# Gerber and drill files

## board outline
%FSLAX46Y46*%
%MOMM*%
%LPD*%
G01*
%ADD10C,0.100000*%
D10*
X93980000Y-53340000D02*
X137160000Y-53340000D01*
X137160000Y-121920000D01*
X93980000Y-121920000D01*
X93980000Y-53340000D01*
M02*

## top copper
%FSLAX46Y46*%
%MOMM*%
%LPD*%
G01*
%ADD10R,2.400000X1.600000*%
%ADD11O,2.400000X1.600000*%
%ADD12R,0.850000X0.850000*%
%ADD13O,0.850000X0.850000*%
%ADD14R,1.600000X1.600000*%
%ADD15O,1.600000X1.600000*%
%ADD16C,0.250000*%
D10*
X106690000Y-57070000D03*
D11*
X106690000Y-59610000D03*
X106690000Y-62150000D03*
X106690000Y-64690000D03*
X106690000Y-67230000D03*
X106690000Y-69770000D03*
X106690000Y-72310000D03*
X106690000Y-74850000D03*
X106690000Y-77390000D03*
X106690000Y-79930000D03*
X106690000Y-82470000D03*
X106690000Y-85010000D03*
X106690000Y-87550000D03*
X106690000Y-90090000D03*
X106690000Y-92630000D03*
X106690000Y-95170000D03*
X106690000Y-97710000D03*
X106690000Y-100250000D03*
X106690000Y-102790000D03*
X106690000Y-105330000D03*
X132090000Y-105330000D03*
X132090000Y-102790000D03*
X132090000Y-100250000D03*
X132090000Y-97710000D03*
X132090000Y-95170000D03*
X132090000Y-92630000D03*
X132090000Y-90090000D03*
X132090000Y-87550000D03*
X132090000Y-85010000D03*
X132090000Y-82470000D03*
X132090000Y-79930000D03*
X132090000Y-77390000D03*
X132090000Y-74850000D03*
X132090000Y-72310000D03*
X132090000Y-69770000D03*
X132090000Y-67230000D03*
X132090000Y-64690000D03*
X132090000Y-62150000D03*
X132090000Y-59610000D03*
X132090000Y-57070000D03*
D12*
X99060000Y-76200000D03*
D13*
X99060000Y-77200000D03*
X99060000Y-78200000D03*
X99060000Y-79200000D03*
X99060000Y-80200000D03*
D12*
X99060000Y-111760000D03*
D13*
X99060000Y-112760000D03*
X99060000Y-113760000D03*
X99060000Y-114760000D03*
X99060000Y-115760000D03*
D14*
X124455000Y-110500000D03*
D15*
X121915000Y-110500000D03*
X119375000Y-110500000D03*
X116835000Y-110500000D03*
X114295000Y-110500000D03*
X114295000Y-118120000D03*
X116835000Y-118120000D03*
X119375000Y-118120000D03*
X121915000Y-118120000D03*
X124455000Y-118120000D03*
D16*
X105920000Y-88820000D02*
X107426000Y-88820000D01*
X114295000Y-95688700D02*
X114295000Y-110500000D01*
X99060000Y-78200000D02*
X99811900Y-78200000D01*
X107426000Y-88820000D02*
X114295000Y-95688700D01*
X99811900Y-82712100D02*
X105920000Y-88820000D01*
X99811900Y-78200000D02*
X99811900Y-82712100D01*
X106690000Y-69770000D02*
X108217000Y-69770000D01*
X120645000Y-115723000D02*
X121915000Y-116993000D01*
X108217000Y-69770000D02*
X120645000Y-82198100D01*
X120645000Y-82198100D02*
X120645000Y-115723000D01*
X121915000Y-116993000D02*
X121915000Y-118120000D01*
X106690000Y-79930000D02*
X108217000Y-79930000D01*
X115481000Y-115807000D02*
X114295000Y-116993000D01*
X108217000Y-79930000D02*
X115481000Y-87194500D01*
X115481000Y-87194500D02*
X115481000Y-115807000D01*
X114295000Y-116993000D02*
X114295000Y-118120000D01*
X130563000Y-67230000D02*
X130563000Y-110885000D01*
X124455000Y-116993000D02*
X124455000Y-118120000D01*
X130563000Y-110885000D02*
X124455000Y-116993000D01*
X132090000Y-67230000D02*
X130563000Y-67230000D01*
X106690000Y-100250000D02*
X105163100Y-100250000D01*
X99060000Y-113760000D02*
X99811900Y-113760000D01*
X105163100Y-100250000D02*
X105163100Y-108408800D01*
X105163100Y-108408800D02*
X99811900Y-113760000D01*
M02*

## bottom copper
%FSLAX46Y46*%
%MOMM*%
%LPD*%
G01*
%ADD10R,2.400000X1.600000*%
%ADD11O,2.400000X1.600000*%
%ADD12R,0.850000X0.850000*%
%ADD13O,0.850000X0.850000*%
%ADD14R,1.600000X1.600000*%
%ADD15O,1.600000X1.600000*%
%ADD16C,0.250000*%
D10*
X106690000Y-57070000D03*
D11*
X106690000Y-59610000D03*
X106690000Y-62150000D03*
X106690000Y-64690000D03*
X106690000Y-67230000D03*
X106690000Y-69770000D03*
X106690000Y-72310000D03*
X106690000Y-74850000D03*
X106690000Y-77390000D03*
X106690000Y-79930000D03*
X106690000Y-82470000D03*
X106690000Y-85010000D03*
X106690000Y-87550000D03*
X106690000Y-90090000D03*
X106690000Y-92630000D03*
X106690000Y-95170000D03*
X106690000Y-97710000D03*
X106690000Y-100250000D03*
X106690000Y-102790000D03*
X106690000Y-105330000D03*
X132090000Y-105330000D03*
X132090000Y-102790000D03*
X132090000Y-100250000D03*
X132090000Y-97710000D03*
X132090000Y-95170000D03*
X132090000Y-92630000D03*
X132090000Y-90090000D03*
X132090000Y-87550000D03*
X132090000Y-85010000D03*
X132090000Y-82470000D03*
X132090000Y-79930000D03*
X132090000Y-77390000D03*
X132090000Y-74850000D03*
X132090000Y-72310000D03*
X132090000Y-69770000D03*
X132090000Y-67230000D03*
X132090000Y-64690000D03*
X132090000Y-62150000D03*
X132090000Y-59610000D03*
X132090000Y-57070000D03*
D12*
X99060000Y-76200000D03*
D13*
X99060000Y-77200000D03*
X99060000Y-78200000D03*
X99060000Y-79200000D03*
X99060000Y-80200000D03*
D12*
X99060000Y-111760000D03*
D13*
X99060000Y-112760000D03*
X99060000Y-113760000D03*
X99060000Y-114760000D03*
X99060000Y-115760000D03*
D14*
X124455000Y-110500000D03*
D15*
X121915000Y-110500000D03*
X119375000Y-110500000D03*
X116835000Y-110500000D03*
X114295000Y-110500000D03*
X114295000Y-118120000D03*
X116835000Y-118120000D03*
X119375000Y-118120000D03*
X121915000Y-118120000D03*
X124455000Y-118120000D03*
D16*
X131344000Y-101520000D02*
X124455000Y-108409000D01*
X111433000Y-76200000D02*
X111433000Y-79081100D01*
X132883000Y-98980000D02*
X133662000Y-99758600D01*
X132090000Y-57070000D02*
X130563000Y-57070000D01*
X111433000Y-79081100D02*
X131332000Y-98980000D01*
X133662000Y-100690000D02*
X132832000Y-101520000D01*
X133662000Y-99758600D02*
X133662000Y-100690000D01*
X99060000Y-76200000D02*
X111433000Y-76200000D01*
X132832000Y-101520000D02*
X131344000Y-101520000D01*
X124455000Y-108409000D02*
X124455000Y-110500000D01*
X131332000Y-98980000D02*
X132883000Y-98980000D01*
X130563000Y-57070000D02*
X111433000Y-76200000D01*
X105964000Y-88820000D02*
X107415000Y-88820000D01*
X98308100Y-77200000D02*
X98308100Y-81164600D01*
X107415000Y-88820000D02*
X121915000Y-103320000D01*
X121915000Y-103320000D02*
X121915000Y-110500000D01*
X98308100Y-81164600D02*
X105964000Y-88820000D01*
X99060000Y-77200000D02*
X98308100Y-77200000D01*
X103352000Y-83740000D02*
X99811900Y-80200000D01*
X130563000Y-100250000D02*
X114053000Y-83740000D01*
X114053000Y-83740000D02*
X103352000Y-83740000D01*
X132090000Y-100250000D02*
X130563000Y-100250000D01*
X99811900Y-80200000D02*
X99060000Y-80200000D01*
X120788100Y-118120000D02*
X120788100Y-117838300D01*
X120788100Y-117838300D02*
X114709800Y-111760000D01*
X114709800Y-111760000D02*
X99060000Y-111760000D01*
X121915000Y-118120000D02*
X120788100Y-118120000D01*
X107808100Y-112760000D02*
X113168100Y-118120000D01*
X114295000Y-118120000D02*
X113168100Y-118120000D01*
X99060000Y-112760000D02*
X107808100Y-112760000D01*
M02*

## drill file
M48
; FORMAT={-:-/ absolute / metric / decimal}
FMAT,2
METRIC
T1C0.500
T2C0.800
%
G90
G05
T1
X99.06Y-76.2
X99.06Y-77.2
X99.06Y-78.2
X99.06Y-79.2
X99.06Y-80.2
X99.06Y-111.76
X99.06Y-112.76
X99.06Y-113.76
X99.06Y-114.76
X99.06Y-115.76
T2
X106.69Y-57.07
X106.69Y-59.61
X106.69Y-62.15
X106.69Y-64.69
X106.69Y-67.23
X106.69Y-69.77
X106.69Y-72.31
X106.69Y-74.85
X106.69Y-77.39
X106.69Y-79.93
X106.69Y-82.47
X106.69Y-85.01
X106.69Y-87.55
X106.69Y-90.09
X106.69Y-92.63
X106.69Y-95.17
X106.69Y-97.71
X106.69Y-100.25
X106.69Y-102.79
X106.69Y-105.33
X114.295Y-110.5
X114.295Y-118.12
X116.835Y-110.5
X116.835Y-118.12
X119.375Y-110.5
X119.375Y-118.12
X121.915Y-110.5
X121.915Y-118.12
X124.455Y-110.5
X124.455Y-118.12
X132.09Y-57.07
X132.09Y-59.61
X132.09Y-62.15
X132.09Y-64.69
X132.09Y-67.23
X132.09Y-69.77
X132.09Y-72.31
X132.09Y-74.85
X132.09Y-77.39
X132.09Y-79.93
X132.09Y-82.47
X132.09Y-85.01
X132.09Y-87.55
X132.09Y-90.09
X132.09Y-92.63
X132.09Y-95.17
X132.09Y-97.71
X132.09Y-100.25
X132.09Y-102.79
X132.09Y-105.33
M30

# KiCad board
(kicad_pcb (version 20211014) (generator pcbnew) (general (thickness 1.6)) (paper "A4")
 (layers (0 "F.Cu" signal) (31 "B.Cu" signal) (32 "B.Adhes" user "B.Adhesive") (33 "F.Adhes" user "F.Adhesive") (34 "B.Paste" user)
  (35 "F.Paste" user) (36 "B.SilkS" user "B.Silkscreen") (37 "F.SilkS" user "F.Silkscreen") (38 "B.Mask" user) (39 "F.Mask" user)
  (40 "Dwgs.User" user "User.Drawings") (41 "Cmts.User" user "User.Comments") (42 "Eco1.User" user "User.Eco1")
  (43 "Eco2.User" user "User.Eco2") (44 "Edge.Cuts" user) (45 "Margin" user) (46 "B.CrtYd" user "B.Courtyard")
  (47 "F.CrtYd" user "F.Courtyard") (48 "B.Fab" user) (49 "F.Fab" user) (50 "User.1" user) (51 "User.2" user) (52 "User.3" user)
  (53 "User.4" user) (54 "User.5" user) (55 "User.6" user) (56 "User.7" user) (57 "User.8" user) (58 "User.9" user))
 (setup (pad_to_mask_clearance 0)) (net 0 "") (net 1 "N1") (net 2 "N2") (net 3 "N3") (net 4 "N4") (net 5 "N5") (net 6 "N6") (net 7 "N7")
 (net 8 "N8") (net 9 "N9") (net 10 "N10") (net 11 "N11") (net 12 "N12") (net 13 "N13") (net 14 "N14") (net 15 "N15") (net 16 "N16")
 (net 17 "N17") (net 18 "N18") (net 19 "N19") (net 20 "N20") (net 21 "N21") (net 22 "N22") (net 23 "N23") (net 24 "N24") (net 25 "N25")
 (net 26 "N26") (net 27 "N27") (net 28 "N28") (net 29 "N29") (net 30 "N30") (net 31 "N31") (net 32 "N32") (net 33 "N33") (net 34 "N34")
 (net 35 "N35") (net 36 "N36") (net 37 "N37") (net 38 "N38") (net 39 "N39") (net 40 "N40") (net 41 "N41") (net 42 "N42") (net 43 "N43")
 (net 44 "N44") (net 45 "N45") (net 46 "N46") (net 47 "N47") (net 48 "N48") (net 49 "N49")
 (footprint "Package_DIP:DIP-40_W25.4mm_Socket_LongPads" (layer "F.Cu") (at 106.69 57.07)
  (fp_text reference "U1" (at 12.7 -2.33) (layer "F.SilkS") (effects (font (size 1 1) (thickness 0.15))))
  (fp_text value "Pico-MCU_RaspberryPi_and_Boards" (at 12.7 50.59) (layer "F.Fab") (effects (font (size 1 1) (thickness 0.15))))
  (pad "1" thru_hole rect (at 0 0) (size 2.4 1.6) (drill 0.8) (layers *.Cu *.Mask) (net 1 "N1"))
  (pad "2" thru_hole oval (at 0 2.54) (size 2.4 1.6) (drill 0.8) (layers *.Cu *.Mask) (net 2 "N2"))
  (pad "3" thru_hole oval (at 0 5.08) (size 2.4 1.6) (drill 0.8) (layers *.Cu *.Mask) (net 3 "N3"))
  (pad "4" thru_hole oval (at 0 7.62) (size 2.4 1.6) (drill 0.8) (layers *.Cu *.Mask) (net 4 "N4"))
  (pad "5" thru_hole oval (at 0 10.16) (size 2.4 1.6) (drill 0.8) (layers *.Cu *.Mask) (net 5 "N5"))
  (pad "6" thru_hole oval (at 0 12.7) (size 2.4 1.6) (drill 0.8) (layers *.Cu *.Mask) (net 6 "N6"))
  (pad "7" thru_hole oval (at 0 15.24) (size 2.4 1.6) (drill 0.8) (layers *.Cu *.Mask) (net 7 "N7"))
  (pad "8" thru_hole oval (at 0 17.78) (size 2.4 1.6) (drill 0.8) (layers *.Cu *.Mask) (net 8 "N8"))
  (pad "9" thru_hole oval (at 0 20.32) (size 2.4 1.6) (drill 0.8) (layers *.Cu *.Mask) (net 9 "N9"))
  (pad "10" thru_hole oval (at 0 22.86) (size 2.4 1.6) (drill 0.8) (layers *.Cu *.Mask) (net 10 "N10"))
  (pad "11" thru_hole oval (at 0 25.4) (size 2.4 1.6) (drill 0.8) (layers *.Cu *.Mask) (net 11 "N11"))
  (pad "12" thru_hole oval (at 0 27.94) (size 2.4 1.6) (drill 0.8) (layers *.Cu *.Mask) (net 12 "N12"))
  (pad "13" thru_hole oval (at 0 30.48) (size 2.4 1.6) (drill 0.8) (layers *.Cu *.Mask) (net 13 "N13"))
  (pad "14" thru_hole oval (at 0 33.02) (size 2.4 1.6) (drill 0.8) (layers *.Cu *.Mask) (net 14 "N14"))
  (pad "15" thru_hole oval (at 0 35.56) (size 2.4 1.6) (drill 0.8) (layers *.Cu *.Mask) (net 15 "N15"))
  (pad "16" thru_hole oval (at 0 38.1) (size 2.4 1.6) (drill 0.8) (layers *.Cu *.Mask) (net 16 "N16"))
  (pad "17" thru_hole oval (at 0 40.64) (size 2.4 1.6) (drill 0.8) (layers *.Cu *.Mask) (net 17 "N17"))
  (pad "18" thru_hole oval (at 0 43.18) (size 2.4 1.6) (drill 0.8) (layers *.Cu *.Mask) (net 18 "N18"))
  (pad "19" thru_hole oval (at 0 45.72) (size 2.4 1.6) (drill 0.8) (layers *.Cu *.Mask) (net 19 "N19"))
  (pad "20" thru_hole oval (at 0 48.26) (size 2.4 1.6) (drill 0.8) (layers *.Cu *.Mask) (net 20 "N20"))
  (pad "21" thru_hole oval (at 25.4 48.26) (size 2.4 1.6) (drill 0.8) (layers *.Cu *.Mask) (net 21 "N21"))
  (pad "22" thru_hole oval (at 25.4 45.72) (size 2.4 1.6) (drill 0.8) (layers *.Cu *.Mask) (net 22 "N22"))
  (pad "23" thru_hole oval (at 25.4 43.18) (size 2.4 1.6) (drill 0.8) (layers *.Cu *.Mask) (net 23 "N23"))
  (pad "24" thru_hole oval (at 25.4 40.64) (size 2.4 1.6) (drill 0.8) (layers *.Cu *.Mask) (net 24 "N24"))
  (pad "25" thru_hole oval (at 25.4 38.1) (size 2.4 1.6) (drill 0.8) (layers *.Cu *.Mask) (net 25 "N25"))
  (pad "26" thru_hole oval (at 25.4 35.56) (size 2.4 1.6) (drill 0.8) (layers *.Cu *.Mask) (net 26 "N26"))
  (pad "27" thru_hole oval (at 25.4 33.02) (size 2.4 1.6) (drill 0.8) (layers *.Cu *.Mask) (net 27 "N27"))
  (pad "28" thru_hole oval (at 25.4 30.48) (size 2.4 1.6) (drill 0.8) (layers *.Cu *.Mask) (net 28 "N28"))
  (pad "29" thru_hole oval (at 25.4 27.94) (size 2.4 1.6) (drill 0.8) (layers *.Cu *.Mask) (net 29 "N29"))
  (pad "30" thru_hole oval (at 25.4 25.4) (size 2.4 1.6) (drill 0.8) (layers *.Cu *.Mask) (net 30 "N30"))
  (pad "31" thru_hole oval (at 25.4 22.86) (size 2.4 1.6) (drill 0.8) (layers *.Cu *.Mask) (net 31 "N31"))
  (pad "32" thru_hole oval (at 25.4 20.32) (size 2.4 1.6) (drill 0.8) (layers *.Cu *.Mask) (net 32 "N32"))
  (pad "33" thru_hole oval (at 25.4 17.78) (size 2.4 1.6) (drill 0.8) (layers *.Cu *.Mask) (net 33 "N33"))
  (pad "34" thru_hole oval (at 25.4 15.24) (size 2.4 1.6) (drill 0.8) (layers *.Cu *.Mask) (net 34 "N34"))
  (pad "35" thru_hole oval (at 25.4 12.7) (size 2.4 1.6) (drill 0.8) (layers *.Cu *.Mask) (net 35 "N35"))
  (pad "36" thru_hole oval (at 25.4 10.16) (size 2.4 1.6) (drill 0.8) (layers *.Cu *.Mask) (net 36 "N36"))
  (pad "37" thru_hole oval (at 25.4 7.62) (size 2.4 1.6) (drill 0.8) (layers *.Cu *.Mask) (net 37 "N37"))
  (pad "38" thru_hole oval (at 25.4 5.08) (size 2.4 1.6) (drill 0.8) (layers *.Cu *.Mask) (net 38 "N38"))
  (pad "39" thru_hole oval (at 25.4 2.54) (size 2.4 1.6) (drill 0.8) (layers *.Cu *.Mask) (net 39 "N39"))
  (pad "40" thru_hole oval (at 25.4 0) (size 2.4 1.6) (drill 0.8) (layers *.Cu *.Mask) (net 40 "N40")))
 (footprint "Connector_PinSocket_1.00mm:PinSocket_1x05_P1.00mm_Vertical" (layer "F.Cu") (at 99.06 76.2)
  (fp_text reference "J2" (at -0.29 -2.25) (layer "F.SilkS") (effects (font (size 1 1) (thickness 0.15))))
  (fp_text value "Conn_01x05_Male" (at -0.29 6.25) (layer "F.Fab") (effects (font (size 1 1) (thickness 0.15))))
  (pad "1" thru_hole rect (at 0 0) (size 0.85 0.85) (drill 0.5) (layers *.Cu *.Mask) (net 40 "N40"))
  (pad "2" thru_hole oval (at 0 1) (size 0.85 0.85) (drill 0.5) (layers *.Cu *.Mask) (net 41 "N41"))
  (pad "3" thru_hole oval (at 0 2) (size 0.85 0.85) (drill 0.5) (layers *.Cu *.Mask) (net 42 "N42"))
  (pad "4" thru_hole oval (at 0 3) (size 0.85 0.85) (drill 0.5) (layers *.Cu *.Mask) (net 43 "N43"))
  (pad "5" thru_hole oval (at 0 4) (size 0.85 0.85) (drill 0.5) (layers *.Cu *.Mask) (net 23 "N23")))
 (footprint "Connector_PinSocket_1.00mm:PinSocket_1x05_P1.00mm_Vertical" (layer "F.Cu") (at 99.06 111.76)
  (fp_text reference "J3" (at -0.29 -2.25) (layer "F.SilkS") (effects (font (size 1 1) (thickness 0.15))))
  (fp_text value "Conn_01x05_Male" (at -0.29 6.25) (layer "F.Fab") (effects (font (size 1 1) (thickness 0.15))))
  (pad "1" thru_hole rect (at 0 0) (size 0.85 0.85) (drill 0.5) (layers *.Cu *.Mask) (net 6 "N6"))
  (pad "2" thru_hole oval (at 0 1) (size 0.85 0.85) (drill 0.5) (layers *.Cu *.Mask) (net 10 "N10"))
  (pad "3" thru_hole oval (at 0 2) (size 0.85 0.85) (drill 0.5) (layers *.Cu *.Mask) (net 18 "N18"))
  (pad "4" thru_hole oval (at 0 3) (size 0.85 0.85) (drill 0.5) (layers *.Cu *.Mask) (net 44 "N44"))
  (pad "5" thru_hole oval (at 0 4) (size 0.85 0.85) (drill 0.5) (layers *.Cu *.Mask) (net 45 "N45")))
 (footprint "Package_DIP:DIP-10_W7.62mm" (layer "F.Cu") (at 124.455 110.5 -90)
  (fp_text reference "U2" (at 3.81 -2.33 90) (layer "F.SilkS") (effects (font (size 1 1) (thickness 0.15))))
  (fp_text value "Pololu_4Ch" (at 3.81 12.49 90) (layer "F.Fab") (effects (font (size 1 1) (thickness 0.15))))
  (pad "1" thru_hole rect (at 0 0 270) (size 1.6 1.6) (drill 0.8) (layers *.Cu *.Mask) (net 40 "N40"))
  (pad "2" thru_hole oval (at 0 2.54 270) (size 1.6 1.6) (drill 0.8) (layers *.Cu *.Mask) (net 41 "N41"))
  (pad "3" thru_hole oval (at 0 5.08 270) (size 1.6 1.6) (drill 0.8) (layers *.Cu *.Mask) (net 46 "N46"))
  (pad "4" thru_hole oval (at 0 7.62 270) (size 1.6 1.6) (drill 0.8) (layers *.Cu *.Mask) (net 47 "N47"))
  (pad "5" thru_hole oval (at 0 10.16 270) (size 1.6 1.6) (drill 0.8) (layers *.Cu *.Mask) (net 42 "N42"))
  (pad "6" thru_hole oval (at 7.62 10.16 270) (size 1.6 1.6) (drill 0.8) (layers *.Cu *.Mask) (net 10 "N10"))
  (pad "7" thru_hole oval (at 7.62 7.62 270) (size 1.6 1.6) (drill 0.8) (layers *.Cu *.Mask) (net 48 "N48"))
  (pad "8" thru_hole oval (at 7.62 5.08 270) (size 1.6 1.6) (drill 0.8) (layers *.Cu *.Mask) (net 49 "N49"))
  (pad "9" thru_hole oval (at 7.62 2.54 270) (size 1.6 1.6) (drill 0.8) (layers *.Cu *.Mask) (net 6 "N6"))
  (pad "10" thru_hole oval (at 7.62 0 270) (size 1.6 1.6) (drill 0.8) (layers *.Cu *.Mask) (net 36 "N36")))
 (gr_rect (start 93.98 53.34) (end 137.16 121.92) (layer "Edge.Cuts") (width 0.1) (fill none))
 (segment (start 131.344 101.52) (end 124.455 108.409) (width 0.25) (layer "B.Cu") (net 40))
 (segment (start 111.433 76.2) (end 111.433 79.0811) (width 0.25) (layer "B.Cu") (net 40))
 (segment (start 132.883 98.98) (end 133.662 99.7586) (width 0.25) (layer "B.Cu") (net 40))
 (segment (start 132.09 57.07) (end 130.563 57.07) (width 0.25) (layer "B.Cu") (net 40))
 (segment (start 111.433 79.0811) (end 131.332 98.98) (width 0.25) (layer "B.Cu") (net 40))
 (segment (start 133.662 100.69) (end 132.832 101.52) (width 0.25) (layer "B.Cu") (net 40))
 (segment (start 133.662 99.7586) (end 133.662 100.69) (width 0.25) (layer "B.Cu") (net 40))
 (segment (start 99.06 76.2) (end 111.433 76.2) (width 0.25) (layer "B.Cu") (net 40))
 (segment (start 132.832 101.52) (end 131.344 101.52) (width 0.25) (layer "B.Cu") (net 40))
 (segment (start 124.455 108.409) (end 124.455 110.5) (width 0.25) (layer "B.Cu") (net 40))
 (segment (start 131.332 98.98) (end 132.883 98.98) (width 0.25) (layer "B.Cu") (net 40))
 (segment (start 130.563 57.07) (end 111.433 76.2) (width 0.25) (layer "B.Cu") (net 40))
 (segment (start 105.964 88.82) (end 107.415 88.82) (width 0.25) (layer "B.Cu") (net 41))
 (segment (start 98.3081 77.2) (end 98.3081 81.1646) (width 0.25) (layer "B.Cu") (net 41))
 (segment (start 107.415 88.82) (end 121.915 103.32) (width 0.25) (layer "B.Cu") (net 41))
 (segment (start 121.915 103.32) (end 121.915 110.5) (width 0.25) (layer "B.Cu") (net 41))
 (segment (start 98.3081 81.1646) (end 105.964 88.82) (width 0.25) (layer "B.Cu") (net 41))
 (segment (start 99.06 77.2) (end 98.3081 77.2) (width 0.25) (layer "B.Cu") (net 41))
 (segment (start 105.92 88.82) (end 107.426 88.82) (width 0.25) (layer "F.Cu") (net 42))
 (segment (start 114.295 95.6887) (end 114.295 110.5) (width 0.25) (layer "F.Cu") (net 42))
 (segment (start 99.06 78.2) (end 99.8119 78.2) (width 0.25) (layer "F.Cu") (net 42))
 (segment (start 107.426 88.82) (end 114.295 95.6887) (width 0.25) (layer "F.Cu") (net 42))
 (segment (start 99.8119 82.7121) (end 105.92 88.82) (width 0.25) (layer "F.Cu") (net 42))
 (segment (start 99.8119 78.2) (end 99.8119 82.7121) (width 0.25) (layer "F.Cu") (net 42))
 (segment (start 103.352 83.74) (end 99.8119 80.2) (width 0.25) (layer "B.Cu") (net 23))
 (segment (start 130.563 100.25) (end 114.053 83.74) (width 0.25) (layer "B.Cu") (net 23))
 (segment (start 114.053 83.74) (end 103.352 83.74) (width 0.25) (layer "B.Cu") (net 23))
 (segment (start 132.09 100.25) (end 130.563 100.25) (width 0.25) (layer "B.Cu") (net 23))
 (segment (start 99.8119 80.2) (end 99.06 80.2) (width 0.25) (layer "B.Cu") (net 23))
 (segment (start 106.69 69.77) (end 108.217 69.77) (width 0.25) (layer "F.Cu") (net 6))
 (segment (start 120.645 115.723) (end 121.915 116.993) (width 0.25) (layer "F.Cu") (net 6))
 (segment (start 108.217 69.77) (end 120.645 82.1981) (width 0.25) (layer "F.Cu") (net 6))
 (segment (start 120.645 82.1981) (end 120.645 115.723) (width 0.25) (layer "F.Cu") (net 6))
 (segment (start 121.915 116.993) (end 121.915 118.12) (width 0.25) (layer "F.Cu") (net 6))
 (segment (start 120.7881 118.12) (end 120.7881 117.8383) (width 0.25) (layer "B.Cu") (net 6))
 (segment (start 120.7881 117.8383) (end 114.7098 111.76) (width 0.25) (layer "B.Cu") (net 6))
 (segment (start 114.7098 111.76) (end 99.06 111.76) (width 0.25) (layer "B.Cu") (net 6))
 (segment (start 121.915 118.12) (end 120.7881 118.12) (width 0.25) (layer "B.Cu") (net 6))
 (segment (start 106.69 79.93) (end 108.217 79.93) (width 0.25) (layer "F.Cu") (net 10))
 (segment (start 115.481 115.807) (end 114.295 116.993) (width 0.25) (layer "F.Cu") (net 10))
 (segment (start 108.217 79.93) (end 115.481 87.1945) (width 0.25) (layer "F.Cu") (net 10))
 (segment (start 115.481 87.1945) (end 115.481 115.807) (width 0.25) (layer "F.Cu") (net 10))
 (segment (start 114.295 116.993) (end 114.295 118.12) (width 0.25) (layer "F.Cu") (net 10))
 (segment (start 107.8081 112.76) (end 113.1681 118.12) (width 0.25) (layer "B.Cu") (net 10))
 (segment (start 114.295 118.12) (end 113.1681 118.12) (width 0.25) (layer "B.Cu") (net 10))
 (segment (start 99.06 112.76) (end 107.8081 112.76) (width 0.25) (layer "B.Cu") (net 10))
 (segment (start 130.563 67.23) (end 130.563 110.885) (width 0.25) (layer "F.Cu") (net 36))
 (segment (start 124.455 116.993) (end 124.455 118.12) (width 0.25) (layer "F.Cu") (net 36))
 (segment (start 130.563 110.885) (end 124.455 116.993) (width 0.25) (layer "F.Cu") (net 36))
 (segment (start 132.09 67.23) (end 130.563 67.23) (width 0.25) (layer "F.Cu") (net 36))
 (segment (start 106.69 100.25) (end 105.1631 100.25) (width 0.25) (layer "F.Cu") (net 18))
 (segment (start 99.06 113.76) (end 99.8119 113.76) (width 0.25) (layer "F.Cu") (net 18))
 (segment (start 105.1631 100.25) (end 105.1631 108.4088) (width 0.25) (layer "F.Cu") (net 18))
 (segment (start 105.1631 108.4088) (end 99.8119 113.76) (width 0.25) (layer "F.Cu") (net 18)))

